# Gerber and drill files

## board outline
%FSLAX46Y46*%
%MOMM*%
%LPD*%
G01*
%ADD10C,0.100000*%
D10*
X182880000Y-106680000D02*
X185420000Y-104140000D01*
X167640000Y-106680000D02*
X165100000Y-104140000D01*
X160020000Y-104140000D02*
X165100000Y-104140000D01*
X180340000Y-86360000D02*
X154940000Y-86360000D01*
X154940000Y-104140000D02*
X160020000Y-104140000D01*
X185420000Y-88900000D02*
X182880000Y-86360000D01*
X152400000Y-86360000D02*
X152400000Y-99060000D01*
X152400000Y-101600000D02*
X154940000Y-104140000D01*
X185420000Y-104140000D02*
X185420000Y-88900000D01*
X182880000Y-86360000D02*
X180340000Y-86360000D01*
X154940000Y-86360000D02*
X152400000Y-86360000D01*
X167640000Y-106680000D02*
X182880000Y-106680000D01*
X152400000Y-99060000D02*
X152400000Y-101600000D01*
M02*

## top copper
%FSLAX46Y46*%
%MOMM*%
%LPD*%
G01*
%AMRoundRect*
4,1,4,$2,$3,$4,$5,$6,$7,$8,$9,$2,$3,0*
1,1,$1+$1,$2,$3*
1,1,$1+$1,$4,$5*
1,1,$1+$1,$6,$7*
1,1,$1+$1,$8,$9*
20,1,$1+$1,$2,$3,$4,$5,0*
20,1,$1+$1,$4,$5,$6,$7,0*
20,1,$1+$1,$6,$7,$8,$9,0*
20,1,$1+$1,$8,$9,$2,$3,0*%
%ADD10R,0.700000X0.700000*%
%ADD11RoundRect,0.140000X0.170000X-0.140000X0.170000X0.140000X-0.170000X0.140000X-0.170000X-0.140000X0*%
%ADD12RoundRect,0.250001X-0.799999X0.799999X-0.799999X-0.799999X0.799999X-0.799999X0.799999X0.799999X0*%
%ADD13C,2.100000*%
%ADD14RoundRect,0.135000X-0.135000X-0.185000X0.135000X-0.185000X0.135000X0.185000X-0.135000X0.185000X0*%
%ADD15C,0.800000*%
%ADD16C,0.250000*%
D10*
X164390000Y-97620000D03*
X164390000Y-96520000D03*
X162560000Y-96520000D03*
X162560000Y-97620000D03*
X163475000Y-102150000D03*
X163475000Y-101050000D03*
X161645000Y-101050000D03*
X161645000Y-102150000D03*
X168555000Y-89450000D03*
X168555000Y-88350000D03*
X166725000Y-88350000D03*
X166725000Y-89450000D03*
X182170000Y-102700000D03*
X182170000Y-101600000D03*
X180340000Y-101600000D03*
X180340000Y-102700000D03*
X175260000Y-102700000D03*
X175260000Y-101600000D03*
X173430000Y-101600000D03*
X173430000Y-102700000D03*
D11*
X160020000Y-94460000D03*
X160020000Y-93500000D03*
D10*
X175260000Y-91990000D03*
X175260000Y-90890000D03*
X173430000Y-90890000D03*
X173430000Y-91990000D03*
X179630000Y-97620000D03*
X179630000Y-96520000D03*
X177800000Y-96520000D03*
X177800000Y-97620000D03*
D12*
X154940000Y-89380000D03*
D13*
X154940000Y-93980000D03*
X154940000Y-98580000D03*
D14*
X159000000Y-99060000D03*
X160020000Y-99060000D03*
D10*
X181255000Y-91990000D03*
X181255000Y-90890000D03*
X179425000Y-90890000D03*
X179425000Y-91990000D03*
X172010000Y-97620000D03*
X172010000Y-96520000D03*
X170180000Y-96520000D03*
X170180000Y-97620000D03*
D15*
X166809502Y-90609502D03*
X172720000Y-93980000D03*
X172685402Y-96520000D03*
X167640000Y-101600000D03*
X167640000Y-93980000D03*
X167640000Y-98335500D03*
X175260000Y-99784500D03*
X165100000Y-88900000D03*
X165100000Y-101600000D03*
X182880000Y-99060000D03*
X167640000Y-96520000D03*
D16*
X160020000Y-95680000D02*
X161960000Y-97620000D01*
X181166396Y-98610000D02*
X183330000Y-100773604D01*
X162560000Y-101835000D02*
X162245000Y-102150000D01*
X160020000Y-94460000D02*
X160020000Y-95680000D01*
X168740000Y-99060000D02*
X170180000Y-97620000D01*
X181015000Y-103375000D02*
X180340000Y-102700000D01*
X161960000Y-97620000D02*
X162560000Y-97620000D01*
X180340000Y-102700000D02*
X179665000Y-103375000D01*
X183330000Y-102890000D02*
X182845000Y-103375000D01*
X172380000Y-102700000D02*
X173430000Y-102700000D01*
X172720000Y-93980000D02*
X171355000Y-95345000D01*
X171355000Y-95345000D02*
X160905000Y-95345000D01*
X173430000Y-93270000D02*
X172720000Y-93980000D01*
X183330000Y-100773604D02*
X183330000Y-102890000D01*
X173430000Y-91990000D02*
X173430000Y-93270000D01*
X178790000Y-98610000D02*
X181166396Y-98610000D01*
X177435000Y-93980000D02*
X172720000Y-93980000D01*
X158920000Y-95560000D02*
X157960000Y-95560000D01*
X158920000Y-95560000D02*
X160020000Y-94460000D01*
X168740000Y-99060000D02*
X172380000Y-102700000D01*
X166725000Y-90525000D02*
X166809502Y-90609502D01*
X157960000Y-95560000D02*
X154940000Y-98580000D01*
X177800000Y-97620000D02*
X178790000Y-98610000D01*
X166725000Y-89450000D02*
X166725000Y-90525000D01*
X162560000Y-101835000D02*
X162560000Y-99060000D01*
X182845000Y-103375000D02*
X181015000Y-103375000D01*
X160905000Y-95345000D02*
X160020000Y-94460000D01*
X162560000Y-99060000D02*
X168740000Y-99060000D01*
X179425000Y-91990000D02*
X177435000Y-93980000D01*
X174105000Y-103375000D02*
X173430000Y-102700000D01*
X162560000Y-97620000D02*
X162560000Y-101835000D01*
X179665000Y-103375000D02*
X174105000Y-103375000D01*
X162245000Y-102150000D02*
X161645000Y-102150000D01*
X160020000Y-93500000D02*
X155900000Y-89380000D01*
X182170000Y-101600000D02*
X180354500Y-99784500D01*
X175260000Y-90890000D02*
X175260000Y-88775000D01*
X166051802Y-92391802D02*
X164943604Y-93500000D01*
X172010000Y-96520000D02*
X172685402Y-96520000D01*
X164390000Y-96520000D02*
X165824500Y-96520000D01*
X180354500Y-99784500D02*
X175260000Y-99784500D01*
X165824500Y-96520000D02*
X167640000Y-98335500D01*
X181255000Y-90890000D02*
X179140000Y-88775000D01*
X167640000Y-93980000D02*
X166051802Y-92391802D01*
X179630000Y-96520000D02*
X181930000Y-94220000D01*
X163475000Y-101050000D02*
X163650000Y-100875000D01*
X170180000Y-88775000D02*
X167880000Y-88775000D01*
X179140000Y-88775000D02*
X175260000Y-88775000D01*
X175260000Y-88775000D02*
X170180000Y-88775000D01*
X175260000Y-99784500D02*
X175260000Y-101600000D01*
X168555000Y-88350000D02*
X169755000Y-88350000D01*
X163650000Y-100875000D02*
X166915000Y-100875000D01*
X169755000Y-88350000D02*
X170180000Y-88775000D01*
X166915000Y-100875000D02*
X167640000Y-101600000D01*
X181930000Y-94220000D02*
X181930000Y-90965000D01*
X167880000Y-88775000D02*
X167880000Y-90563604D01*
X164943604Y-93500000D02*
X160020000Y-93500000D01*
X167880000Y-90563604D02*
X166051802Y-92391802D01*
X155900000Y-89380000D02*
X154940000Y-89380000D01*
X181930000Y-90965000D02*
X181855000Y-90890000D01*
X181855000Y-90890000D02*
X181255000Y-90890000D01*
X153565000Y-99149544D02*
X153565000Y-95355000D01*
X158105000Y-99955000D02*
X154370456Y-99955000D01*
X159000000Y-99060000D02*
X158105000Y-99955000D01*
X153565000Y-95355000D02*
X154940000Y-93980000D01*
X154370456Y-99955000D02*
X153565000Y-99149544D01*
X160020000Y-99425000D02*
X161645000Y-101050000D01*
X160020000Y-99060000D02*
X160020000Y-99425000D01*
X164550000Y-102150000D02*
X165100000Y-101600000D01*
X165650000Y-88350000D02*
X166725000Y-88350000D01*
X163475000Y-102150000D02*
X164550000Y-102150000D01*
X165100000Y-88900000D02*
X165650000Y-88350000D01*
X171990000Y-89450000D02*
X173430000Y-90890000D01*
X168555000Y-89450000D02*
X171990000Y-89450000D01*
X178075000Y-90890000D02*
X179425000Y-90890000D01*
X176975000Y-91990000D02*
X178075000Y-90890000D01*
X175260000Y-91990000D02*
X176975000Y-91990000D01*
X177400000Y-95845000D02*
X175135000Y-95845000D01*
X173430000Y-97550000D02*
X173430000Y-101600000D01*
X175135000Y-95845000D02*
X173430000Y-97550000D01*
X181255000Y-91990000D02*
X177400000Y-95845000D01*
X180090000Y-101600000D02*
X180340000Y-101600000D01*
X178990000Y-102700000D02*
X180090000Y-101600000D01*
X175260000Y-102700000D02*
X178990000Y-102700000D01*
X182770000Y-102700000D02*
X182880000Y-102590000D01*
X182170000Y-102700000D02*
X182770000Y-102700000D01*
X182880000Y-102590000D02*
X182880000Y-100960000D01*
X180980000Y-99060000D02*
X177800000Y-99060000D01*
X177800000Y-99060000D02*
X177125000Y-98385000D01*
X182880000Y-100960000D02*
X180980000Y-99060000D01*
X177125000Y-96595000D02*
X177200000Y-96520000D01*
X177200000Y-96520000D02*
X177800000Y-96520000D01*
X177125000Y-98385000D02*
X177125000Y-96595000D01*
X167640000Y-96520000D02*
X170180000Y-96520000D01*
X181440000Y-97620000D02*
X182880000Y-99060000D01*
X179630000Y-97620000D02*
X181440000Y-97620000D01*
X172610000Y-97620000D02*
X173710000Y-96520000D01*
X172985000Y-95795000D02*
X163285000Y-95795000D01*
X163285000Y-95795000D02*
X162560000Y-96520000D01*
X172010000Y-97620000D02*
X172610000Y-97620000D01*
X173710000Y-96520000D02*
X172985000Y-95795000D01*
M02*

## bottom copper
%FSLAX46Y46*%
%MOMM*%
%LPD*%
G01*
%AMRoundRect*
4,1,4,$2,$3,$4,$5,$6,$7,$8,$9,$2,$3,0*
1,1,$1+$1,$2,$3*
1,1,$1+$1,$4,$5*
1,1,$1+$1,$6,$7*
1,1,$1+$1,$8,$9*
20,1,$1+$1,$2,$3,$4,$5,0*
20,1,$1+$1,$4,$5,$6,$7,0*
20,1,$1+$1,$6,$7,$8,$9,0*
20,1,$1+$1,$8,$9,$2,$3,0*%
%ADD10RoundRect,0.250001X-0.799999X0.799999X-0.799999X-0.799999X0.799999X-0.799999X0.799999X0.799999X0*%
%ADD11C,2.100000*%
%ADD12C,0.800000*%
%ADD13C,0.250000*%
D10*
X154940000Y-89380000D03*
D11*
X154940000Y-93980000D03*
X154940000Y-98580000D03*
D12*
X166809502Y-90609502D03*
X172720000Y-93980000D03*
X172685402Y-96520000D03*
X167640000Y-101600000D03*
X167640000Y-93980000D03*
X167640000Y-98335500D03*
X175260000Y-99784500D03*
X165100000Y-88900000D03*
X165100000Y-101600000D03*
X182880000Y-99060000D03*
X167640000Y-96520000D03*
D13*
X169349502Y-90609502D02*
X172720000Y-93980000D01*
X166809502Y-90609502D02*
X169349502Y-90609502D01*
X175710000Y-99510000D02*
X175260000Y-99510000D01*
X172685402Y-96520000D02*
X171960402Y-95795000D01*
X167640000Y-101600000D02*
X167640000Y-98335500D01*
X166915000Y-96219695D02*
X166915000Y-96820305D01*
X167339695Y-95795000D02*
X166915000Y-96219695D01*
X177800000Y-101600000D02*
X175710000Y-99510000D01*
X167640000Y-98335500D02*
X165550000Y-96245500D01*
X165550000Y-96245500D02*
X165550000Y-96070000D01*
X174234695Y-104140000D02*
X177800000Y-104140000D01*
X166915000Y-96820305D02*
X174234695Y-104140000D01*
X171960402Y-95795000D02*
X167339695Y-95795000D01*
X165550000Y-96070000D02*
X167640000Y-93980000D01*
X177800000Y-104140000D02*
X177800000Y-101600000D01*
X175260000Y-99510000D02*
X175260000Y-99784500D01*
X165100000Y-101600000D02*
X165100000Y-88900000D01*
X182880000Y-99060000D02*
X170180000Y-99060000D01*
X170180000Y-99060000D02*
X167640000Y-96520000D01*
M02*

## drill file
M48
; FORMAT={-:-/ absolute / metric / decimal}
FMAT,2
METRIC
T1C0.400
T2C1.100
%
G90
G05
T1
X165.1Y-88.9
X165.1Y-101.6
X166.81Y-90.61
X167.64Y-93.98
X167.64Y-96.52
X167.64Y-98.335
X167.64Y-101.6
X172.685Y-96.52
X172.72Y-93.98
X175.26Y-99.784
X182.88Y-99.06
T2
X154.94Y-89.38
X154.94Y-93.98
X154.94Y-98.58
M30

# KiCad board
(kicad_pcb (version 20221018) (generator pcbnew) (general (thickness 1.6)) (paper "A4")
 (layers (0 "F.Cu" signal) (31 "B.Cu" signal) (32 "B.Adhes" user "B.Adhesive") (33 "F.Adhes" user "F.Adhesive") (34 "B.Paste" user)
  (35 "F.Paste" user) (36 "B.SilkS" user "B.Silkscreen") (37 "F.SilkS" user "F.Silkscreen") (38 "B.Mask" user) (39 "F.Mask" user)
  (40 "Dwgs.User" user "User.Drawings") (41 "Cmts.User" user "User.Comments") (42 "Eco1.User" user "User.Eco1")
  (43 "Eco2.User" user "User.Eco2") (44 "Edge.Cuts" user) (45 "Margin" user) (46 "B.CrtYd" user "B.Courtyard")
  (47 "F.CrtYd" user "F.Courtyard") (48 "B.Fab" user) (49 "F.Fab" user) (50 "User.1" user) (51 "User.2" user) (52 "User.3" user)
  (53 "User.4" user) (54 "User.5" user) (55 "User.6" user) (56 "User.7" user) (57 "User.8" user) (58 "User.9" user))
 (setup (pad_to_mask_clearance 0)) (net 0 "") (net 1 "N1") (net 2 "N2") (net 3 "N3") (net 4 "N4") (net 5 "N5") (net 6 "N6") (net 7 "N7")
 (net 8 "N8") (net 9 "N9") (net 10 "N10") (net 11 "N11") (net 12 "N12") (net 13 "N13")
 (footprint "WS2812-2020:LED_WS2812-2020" (layer "F.Cu") (at 163.475 97.07)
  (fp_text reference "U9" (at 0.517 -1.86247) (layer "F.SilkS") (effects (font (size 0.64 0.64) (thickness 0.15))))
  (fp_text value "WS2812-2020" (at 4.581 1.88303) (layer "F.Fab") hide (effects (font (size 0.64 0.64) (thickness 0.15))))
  (pad "1" smd rect (at 0.915 0.55) (size 0.7 0.7) (layers "F.Cu" "F.Paste" "F.Mask") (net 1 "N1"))
  (pad "2" smd rect (at 0.915 -0.55) (size 0.7 0.7) (layers "F.Cu" "F.Paste" "F.Mask") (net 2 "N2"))
  (pad "3" smd rect (at -0.915 -0.55) (size 0.7 0.7) (layers "F.Cu" "F.Paste" "F.Mask") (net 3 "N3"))
  (pad "4" smd rect (at -0.915 0.55) (size 0.7 0.7) (layers "F.Cu" "F.Paste" "F.Mask") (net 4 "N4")))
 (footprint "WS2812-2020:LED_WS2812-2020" (layer "F.Cu") (at 162.56 101.6)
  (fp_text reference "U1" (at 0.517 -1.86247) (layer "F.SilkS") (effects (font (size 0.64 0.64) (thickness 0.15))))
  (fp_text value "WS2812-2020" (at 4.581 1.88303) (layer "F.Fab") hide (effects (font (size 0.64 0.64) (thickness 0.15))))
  (pad "1" smd rect (at 0.915 0.55) (size 0.7 0.7) (layers "F.Cu" "F.Paste" "F.Mask") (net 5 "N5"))
  (pad "2" smd rect (at 0.915 -0.55) (size 0.7 0.7) (layers "F.Cu" "F.Paste" "F.Mask") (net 2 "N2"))
  (pad "3" smd rect (at -0.915 -0.55) (size 0.7 0.7) (layers "F.Cu" "F.Paste" "F.Mask") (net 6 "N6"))
  (pad "4" smd rect (at -0.915 0.55) (size 0.7 0.7) (layers "F.Cu" "F.Paste" "F.Mask") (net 4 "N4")))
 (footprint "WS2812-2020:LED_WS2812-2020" (layer "F.Cu") (at 167.64 88.9)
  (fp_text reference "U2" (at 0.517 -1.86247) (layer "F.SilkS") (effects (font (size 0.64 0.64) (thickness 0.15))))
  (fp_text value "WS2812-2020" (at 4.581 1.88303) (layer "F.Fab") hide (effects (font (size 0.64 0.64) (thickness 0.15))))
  (pad "1" smd rect (at 0.915 0.55) (size 0.7 0.7) (layers "F.Cu" "F.Paste" "F.Mask") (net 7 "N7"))
  (pad "2" smd rect (at 0.915 -0.55) (size 0.7 0.7) (layers "F.Cu" "F.Paste" "F.Mask") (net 2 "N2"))
  (pad "3" smd rect (at -0.915 -0.55) (size 0.7 0.7) (layers "F.Cu" "F.Paste" "F.Mask") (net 5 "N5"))
  (pad "4" smd rect (at -0.915 0.55) (size 0.7 0.7) (layers "F.Cu" "F.Paste" "F.Mask") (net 4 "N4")))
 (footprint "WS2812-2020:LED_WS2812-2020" (layer "F.Cu") (at 181.255 102.15)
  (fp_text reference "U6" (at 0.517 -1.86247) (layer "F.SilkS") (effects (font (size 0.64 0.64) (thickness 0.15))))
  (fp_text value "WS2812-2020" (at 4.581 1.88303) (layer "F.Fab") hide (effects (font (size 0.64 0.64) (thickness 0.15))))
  (pad "1" smd rect (at 0.915 0.55) (size 0.7 0.7) (layers "F.Cu" "F.Paste" "F.Mask") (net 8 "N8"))
  (pad "2" smd rect (at 0.915 -0.55) (size 0.7 0.7) (layers "F.Cu" "F.Paste" "F.Mask") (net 2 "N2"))
  (pad "3" smd rect (at -0.915 -0.55) (size 0.7 0.7) (layers "F.Cu" "F.Paste" "F.Mask") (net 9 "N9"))
  (pad "4" smd rect (at -0.915 0.55) (size 0.7 0.7) (layers "F.Cu" "F.Paste" "F.Mask") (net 4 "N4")))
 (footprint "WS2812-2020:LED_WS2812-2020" (layer "F.Cu") (at 174.345 102.15)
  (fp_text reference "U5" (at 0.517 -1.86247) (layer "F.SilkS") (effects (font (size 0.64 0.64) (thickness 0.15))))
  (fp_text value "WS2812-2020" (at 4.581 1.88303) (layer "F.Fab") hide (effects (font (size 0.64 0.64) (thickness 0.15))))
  (pad "1" smd rect (at 0.915 0.55) (size 0.7 0.7) (layers "F.Cu" "F.Paste" "F.Mask") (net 9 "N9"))
  (pad "2" smd rect (at 0.915 -0.55) (size 0.7 0.7) (layers "F.Cu" "F.Paste" "F.Mask") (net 2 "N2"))
  (pad "3" smd rect (at -0.915 -0.55) (size 0.7 0.7) (layers "F.Cu" "F.Paste" "F.Mask") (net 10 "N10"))
  (pad "4" smd rect (at -0.915 0.55) (size 0.7 0.7) (layers "F.Cu" "F.Paste" "F.Mask") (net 4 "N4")))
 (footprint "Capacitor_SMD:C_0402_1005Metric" (layer "F.Cu") (at 160.02 93.98 90)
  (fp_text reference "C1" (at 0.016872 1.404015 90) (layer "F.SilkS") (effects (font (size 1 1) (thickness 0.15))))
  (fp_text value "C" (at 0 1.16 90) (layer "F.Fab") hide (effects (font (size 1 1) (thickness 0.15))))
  (pad "1" smd roundrect (at -0.48 0 90) (size 0.56 0.62) (layers "F.Cu" "F.Paste" "F.Mask") (roundrect_rratio 0.25) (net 4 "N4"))
  (pad "2" smd roundrect (at 0.48 0 90) (size 0.56 0.62) (layers "F.Cu" "F.Paste" "F.Mask") (roundrect_rratio 0.25) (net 2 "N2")))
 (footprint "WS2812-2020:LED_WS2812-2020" (layer "F.Cu") (at 174.345 91.44)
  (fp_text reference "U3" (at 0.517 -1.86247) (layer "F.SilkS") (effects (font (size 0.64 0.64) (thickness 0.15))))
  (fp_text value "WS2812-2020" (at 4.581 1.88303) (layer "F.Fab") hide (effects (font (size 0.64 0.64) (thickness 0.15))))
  (pad "1" smd rect (at 0.915 0.55) (size 0.7 0.7) (layers "F.Cu" "F.Paste" "F.Mask") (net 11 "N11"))
  (pad "2" smd rect (at 0.915 -0.55) (size 0.7 0.7) (layers "F.Cu" "F.Paste" "F.Mask") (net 2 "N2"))
  (pad "3" smd rect (at -0.915 -0.55) (size 0.7 0.7) (layers "F.Cu" "F.Paste" "F.Mask") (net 7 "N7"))
  (pad "4" smd rect (at -0.915 0.55) (size 0.7 0.7) (layers "F.Cu" "F.Paste" "F.Mask") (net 4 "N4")))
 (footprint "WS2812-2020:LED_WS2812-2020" (layer "F.Cu") (at 178.715 97.07)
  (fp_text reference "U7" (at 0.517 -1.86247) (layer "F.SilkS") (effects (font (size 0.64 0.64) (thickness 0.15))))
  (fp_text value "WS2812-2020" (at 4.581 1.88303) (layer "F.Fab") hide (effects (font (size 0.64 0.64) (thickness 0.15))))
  (pad "1" smd rect (at 0.915 0.55) (size 0.7 0.7) (layers "F.Cu" "F.Paste" "F.Mask") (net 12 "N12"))
  (pad "2" smd rect (at 0.915 -0.55) (size 0.7 0.7) (layers "F.Cu" "F.Paste" "F.Mask") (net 2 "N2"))
  (pad "3" smd rect (at -0.915 -0.55) (size 0.7 0.7) (layers "F.Cu" "F.Paste" "F.Mask") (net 8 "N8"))
  (pad "4" smd rect (at -0.915 0.55) (size 0.7 0.7) (layers "F.Cu" "F.Paste" "F.Mask") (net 4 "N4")))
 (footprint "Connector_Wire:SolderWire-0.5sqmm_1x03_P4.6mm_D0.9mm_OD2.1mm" (layer "F.Cu") (at 154.94 89.38 -90)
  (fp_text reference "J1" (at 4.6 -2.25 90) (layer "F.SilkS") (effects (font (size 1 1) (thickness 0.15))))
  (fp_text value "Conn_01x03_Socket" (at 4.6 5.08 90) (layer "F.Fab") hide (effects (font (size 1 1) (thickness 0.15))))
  (pad "1" thru_hole roundrect (at 0 0 270) (size 2.1 2.1) (drill 1.1) (layers "*.Cu" "*.Mask") (roundrect_rratio 0.119048) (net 2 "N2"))
  (pad "2" thru_hole circle (at 4.6 0 270) (size 2.1 2.1) (drill 1.1) (layers "*.Cu" "*.Mask") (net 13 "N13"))
  (pad "3" thru_hole circle (at 9.2 0 270) (size 2.1 2.1) (drill 1.1) (layers "*.Cu" "*.Mask") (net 4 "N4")))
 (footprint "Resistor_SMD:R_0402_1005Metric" (layer "F.Cu") (at 159.51 99.06)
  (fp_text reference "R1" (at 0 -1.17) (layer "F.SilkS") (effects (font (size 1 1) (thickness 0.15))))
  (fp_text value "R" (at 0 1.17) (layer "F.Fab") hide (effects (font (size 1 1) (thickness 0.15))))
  (pad "1" smd roundrect (at -0.51 0) (size 0.54 0.64) (layers "F.Cu" "F.Paste" "F.Mask") (roundrect_rratio 0.25) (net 13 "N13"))
  (pad "2" smd roundrect (at 0.51 0) (size 0.54 0.64) (layers "F.Cu" "F.Paste" "F.Mask") (roundrect_rratio 0.25) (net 6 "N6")))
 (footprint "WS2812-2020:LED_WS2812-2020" (layer "F.Cu") (at 180.34 91.44)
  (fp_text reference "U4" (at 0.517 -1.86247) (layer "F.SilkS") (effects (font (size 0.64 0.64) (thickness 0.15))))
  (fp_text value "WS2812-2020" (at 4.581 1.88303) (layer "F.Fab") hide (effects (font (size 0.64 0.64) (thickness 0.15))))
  (pad "1" smd rect (at 0.915 0.55) (size 0.7 0.7) (layers "F.Cu" "F.Paste" "F.Mask") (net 10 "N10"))
  (pad "2" smd rect (at 0.915 -0.55) (size 0.7 0.7) (layers "F.Cu" "F.Paste" "F.Mask") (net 2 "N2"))
  (pad "3" smd rect (at -0.915 -0.55) (size 0.7 0.7) (layers "F.Cu" "F.Paste" "F.Mask") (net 11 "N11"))
  (pad "4" smd rect (at -0.915 0.55) (size 0.7 0.7) (layers "F.Cu" "F.Paste" "F.Mask") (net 4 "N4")))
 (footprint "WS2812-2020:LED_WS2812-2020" (layer "F.Cu") (at 171.095 97.07)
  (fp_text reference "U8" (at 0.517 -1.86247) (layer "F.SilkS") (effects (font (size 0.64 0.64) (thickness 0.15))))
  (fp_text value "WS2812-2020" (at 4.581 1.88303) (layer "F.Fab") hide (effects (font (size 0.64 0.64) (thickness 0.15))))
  (pad "1" smd rect (at 0.915 0.55) (size 0.7 0.7) (layers "F.Cu" "F.Paste" "F.Mask") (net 3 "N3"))
  (pad "2" smd rect (at 0.915 -0.55) (size 0.7 0.7) (layers "F.Cu" "F.Paste" "F.Mask") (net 2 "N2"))
  (pad "3" smd rect (at -0.915 -0.55) (size 0.7 0.7) (layers "F.Cu" "F.Paste" "F.Mask") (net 12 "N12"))
  (pad "4" smd rect (at -0.915 0.55) (size 0.7 0.7) (layers "F.Cu" "F.Paste" "F.Mask") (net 4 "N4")))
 (gr_line (start 182.88 106.68) (end 185.42 104.14) (stroke (width 0.1) (type default)) (layer "Edge.Cuts"))
 (gr_line (start 167.64 106.68) (end 165.1 104.14) (stroke (width 0.1) (type default)) (layer "Edge.Cuts"))
 (gr_line (start 160.02 104.14) (end 165.1 104.14) (stroke (width 0.1) (type default)) (layer "Edge.Cuts"))
 (gr_line (start 180.34 86.36) (end 154.94 86.36) (stroke (width 0.1) (type default)) (layer "Edge.Cuts"))
 (gr_line (start 154.94 104.14) (end 160.02 104.14) (stroke (width 0.1) (type default)) (layer "Edge.Cuts"))
 (gr_line (start 185.42 88.9) (end 182.88 86.36) (stroke (width 0.1) (type default)) (layer "Edge.Cuts"))
 (gr_line (start 152.4 86.36) (end 152.4 99.06) (stroke (width 0.1) (type default)) (layer "Edge.Cuts"))
 (gr_line (start 152.4 101.6) (end 154.94 104.14) (stroke (width 0.1) (type default)) (layer "Edge.Cuts"))
 (gr_line (start 185.42 104.14) (end 185.42 88.9) (stroke (width 0.1) (type default)) (layer "Edge.Cuts"))
 (gr_line (start 182.88 86.36) (end 180.34 86.36) (stroke (width 0.1) (type default)) (layer "Edge.Cuts"))
 (gr_line (start 154.94 86.36) (end 152.4 86.36) (stroke (width 0.1) (type default)) (layer "Edge.Cuts"))
 (gr_line (start 167.64 106.68) (end 182.88 106.68) (stroke (width 0.1) (type default)) (layer "Edge.Cuts"))
 (gr_line (start 152.4 99.06) (end 152.4 101.6) (stroke (width 0.1) (type default)) (layer "Edge.Cuts"))
 (segment (start 160.02 95.68) (end 161.96 97.62) (width 0.25) (layer "F.Cu") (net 4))
 (segment (start 181.166396 98.61) (end 183.33 100.773604) (width 0.25) (layer "F.Cu") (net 4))
 (segment (start 162.56 101.835) (end 162.245 102.15) (width 0.25) (layer "F.Cu") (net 4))
 (segment (start 160.02 94.46) (end 160.02 95.68) (width 0.25) (layer "F.Cu") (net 4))
 (segment (start 168.74 99.06) (end 170.18 97.62) (width 0.25) (layer "F.Cu") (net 4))
 (segment (start 181.015 103.375) (end 180.34 102.7) (width 0.25) (layer "F.Cu") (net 4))
 (segment (start 161.96 97.62) (end 162.56 97.62) (width 0.25) (layer "F.Cu") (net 4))
 (segment (start 180.34 102.7) (end 179.665 103.375) (width 0.25) (layer "F.Cu") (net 4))
 (segment (start 183.33 102.89) (end 182.845 103.375) (width 0.25) (layer "F.Cu") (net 4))
 (segment (start 172.38 102.7) (end 173.43 102.7) (width 0.25) (layer "F.Cu") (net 4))
 (segment (start 172.72 93.98) (end 171.355 95.345) (width 0.25) (layer "F.Cu") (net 4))
 (segment (start 171.355 95.345) (end 160.905 95.345) (width 0.25) (layer "F.Cu") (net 4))
 (segment (start 173.43 93.27) (end 172.72 93.98) (width 0.25) (layer "F.Cu") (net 4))
 (segment (start 183.33 100.773604) (end 183.33 102.89) (width 0.25) (layer "F.Cu") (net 4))
 (segment (start 173.43 91.99) (end 173.43 93.27) (width 0.25) (layer "F.Cu") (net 4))
 (segment (start 178.79 98.61) (end 181.166396 98.61) (width 0.25) (layer "F.Cu") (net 4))
 (segment (start 177.435 93.98) (end 172.72 93.98) (width 0.25) (layer "F.Cu") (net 4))
 (segment (start 158.92 95.56) (end 157.96 95.56) (width 0.25) (layer "F.Cu") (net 4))
 (segment (start 158.92 95.56) (end 160.02 94.46) (width 0.25) (layer "F.Cu") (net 4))
 (segment (start 168.74 99.06) (end 172.38 102.7) (width 0.25) (layer "F.Cu") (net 4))
 (segment (start 166.725 90.525) (end 166.809502 90.609502) (width 0.25) (layer "F.Cu") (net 4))
 (segment (start 157.96 95.56) (end 154.94 98.58) (width 0.25) (layer "F.Cu") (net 4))
 (segment (start 177.8 97.62) (end 178.79 98.61) (width 0.25) (layer "F.Cu") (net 4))
 (segment (start 166.725 89.45) (end 166.725 90.525) (width 0.25) (layer "F.Cu") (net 4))
 (segment (start 162.56 101.835) (end 162.56 99.06) (width 0.25) (layer "F.Cu") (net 4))
 (segment (start 182.845 103.375) (end 181.015 103.375) (width 0.25) (layer "F.Cu") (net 4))
 (segment (start 160.905 95.345) (end 160.02 94.46) (width 0.25) (layer "F.Cu") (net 4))
 (segment (start 162.56 99.06) (end 168.74 99.06) (width 0.25) (layer "F.Cu") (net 4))
 (segment (start 179.425 91.99) (end 177.435 93.98) (width 0.25) (layer "F.Cu") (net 4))
 (segment (start 174.105 103.375) (end 173.43 102.7) (width 0.25) (layer "F.Cu") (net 4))
 (segment (start 162.56 97.62) (end 162.56 101.835) (width 0.25) (layer "F.Cu") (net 4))
 (segment (start 179.665 103.375) (end 174.105 103.375) (width 0.25) (layer "F.Cu") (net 4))
 (segment (start 162.245 102.15) (end 161.645 102.15) (width 0.25) (layer "F.Cu") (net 4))
 (via (at 166.809502 90.609502) (size 0.8) (drill 0.4) (layers "F.Cu" "B.Cu") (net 4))
 (via (at 172.72 93.98) (size 0.8) (drill 0.4) (layers "F.Cu" "B.Cu") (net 4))
 (segment (start 169.349502 90.609502) (end 172.72 93.98) (width 0.25) (layer "B.Cu") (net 4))
 (segment (start 166.809502 90.609502) (end 169.349502 90.609502) (width 0.25) (layer "B.Cu") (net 4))
 (segment (start 160.02 93.5) (end 155.9 89.38) (width 0.25) (layer "F.Cu") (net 2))
 (segment (start 182.17 101.6) (end 180.3545 99.7845) (width 0.25) (layer "F.Cu") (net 2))
 (segment (start 175.26 90.89) (end 175.26 88.775) (width 0.25) (layer "F.Cu") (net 2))
 (segment (start 166.051802 92.391802) (end 164.943604 93.5) (width 0.25) (layer "F.Cu") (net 2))
 (segment (start 172.01 96.52) (end 172.685402 96.52) (width 0.25) (layer "F.Cu") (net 2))
 (segment (start 164.39 96.52) (end 165.8245 96.52) (width 0.25) (layer "F.Cu") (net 2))
 (segment (start 180.3545 99.7845) (end 175.26 99.7845) (width 0.25) (layer "F.Cu") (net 2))
 (segment (start 165.8245 96.52) (end 167.64 98.3355) (width 0.25) (layer "F.Cu") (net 2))
 (segment (start 181.255 90.89) (end 179.14 88.775) (width 0.25) (layer "F.Cu") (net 2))
 (segment (start 167.64 93.98) (end 166.051802 92.391802) (width 0.25) (layer "F.Cu") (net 2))
 (segment (start 179.63 96.52) (end 181.93 94.22) (width 0.25) (layer "F.Cu") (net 2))
 (segment (start 163.475 101.05) (end 163.65 100.875) (width 0.25) (layer "F.Cu") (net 2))
 (segment (start 170.18 88.775) (end 167.88 88.775) (width 0.25) (layer "F.Cu") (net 2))
 (segment (start 179.14 88.775) (end 175.26 88.775) (width 0.25) (layer "F.Cu") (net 2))
 (segment (start 175.26 88.775) (end 170.18 88.775) (width 0.25) (layer "F.Cu") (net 2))
 (segment (start 175.26 99.7845) (end 175.26 101.6) (width 0.25) (layer "F.Cu") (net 2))
 (segment (start 168.555 88.35) (end 169.755 88.35) (width 0.25) (layer "F.Cu") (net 2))
 (segment (start 163.65 100.875) (end 166.915 100.875) (width 0.25) (layer "F.Cu") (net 2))
 (segment (start 169.755 88.35) (end 170.18 88.775) (width 0.25) (layer "F.Cu") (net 2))
 (segment (start 166.915 100.875) (end 167.64 101.6) (width 0.25) (layer "F.Cu") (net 2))
 (segment (start 181.93 94.22) (end 181.93 90.965) (width 0.25) (layer "F.Cu") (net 2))
 (segment (start 167.88 88.775) (end 167.88 90.563604) (width 0.25) (layer "F.Cu") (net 2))
 (segment (start 164.943604 93.5) (end 160.02 93.5) (width 0.25) (layer "F.Cu") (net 2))
 (segment (start 167.88 90.563604) (end 166.051802 92.391802) (width 0.25) (layer "F.Cu") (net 2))
 (segment (start 155.9 89.38) (end 154.94 89.38) (width 0.25) (layer "F.Cu") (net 2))
 (segment (start 181.93 90.965) (end 181.855 90.89) (width 0.25) (layer "F.Cu") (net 2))
 (segment (start 181.855 90.89) (end 181.255 90.89) (width 0.25) (layer "F.Cu") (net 2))
 (via (at 172.685402 96.52) (size 0.8) (drill 0.4) (layers "F.Cu" "B.Cu") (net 2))
 (via (at 167.64 101.6) (size 0.8) (drill 0.4) (layers "F.Cu" "B.Cu") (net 2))
 (via (at 167.64 93.98) (size 0.8) (drill 0.4) (layers "F.Cu" "B.Cu") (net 2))
 (via (at 167.64 98.3355) (size 0.8) (drill 0.4) (layers "F.Cu" "B.Cu") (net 2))
 (via (at 175.26 99.7845) (size 0.8) (drill 0.4) (layers "F.Cu" "B.Cu") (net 2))
 (segment (start 175.71 99.51) (end 175.26 99.51) (width 0.25) (layer "B.Cu") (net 2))
 (segment (start 172.685402 96.52) (end 171.960402 95.795) (width 0.25) (layer "B.Cu") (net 2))
 (segment (start 167.64 101.6) (end 167.64 98.3355) (width 0.25) (layer "B.Cu") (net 2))
 (segment (start 166.915 96.219695) (end 166.915 96.820305) (width 0.25) (layer "B.Cu") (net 2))
 (segment (start 167.339695 95.795) (end 166.915 96.219695) (width 0.25) (layer "B.Cu") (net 2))
 (segment (start 177.8 101.6) (end 175.71 99.51) (width 0.25) (layer "B.Cu") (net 2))
 (segment (start 167.64 98.3355) (end 165.55 96.2455) (width 0.25) (layer "B.Cu") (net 2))
 (segment (start 165.55 96.2455) (end 165.55 96.07) (width 0.25) (layer "B.Cu") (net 2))
 (segment (start 174.234695 104.14) (end 177.8 104.14) (width 0.25) (layer "B.Cu") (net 2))
 (segment (start 166.915 96.820305) (end 174.234695 104.14) (width 0.25) (layer "B.Cu") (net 2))
 (segment (start 171.960402 95.795) (end 167.339695 95.795) (width 0.25) (layer "B.Cu") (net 2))
 (segment (start 165.55 96.07) (end 167.64 93.98) (width 0.25) (layer "B.Cu") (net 2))
 (segment (start 177.8 104.14) (end 177.8 101.6) (width 0.25) (layer "B.Cu") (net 2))
 (segment (start 175.26 99.51) (end 175.26 99.7845) (width 0.25) (layer "B.Cu") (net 2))
 (segment (start 153.565 99.149544) (end 153.565 95.355) (width 0.25) (layer "F.Cu") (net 13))
 (segment (start 158.105 99.955) (end 154.370456 99.955) (width 0.25) (layer "F.Cu") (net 13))
 (segment (start 159 99.06) (end 158.105 99.955) (width 0.25) (layer "F.Cu") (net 13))
 (segment (start 153.565 95.355) (end 154.94 93.98) (width 0.25) (layer "F.Cu") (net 13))
 (segment (start 154.370456 99.955) (end 153.565 99.149544) (width 0.25) (layer "F.Cu") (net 13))
 (segment (start 160.02 99.425) (end 161.645 101.05) (width 0.25) (layer "F.Cu") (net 6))
 (segment (start 160.02 99.06) (end 160.02 99.425) (width 0.25) (layer "F.Cu") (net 6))
 (segment (start 164.55 102.15) (end 165.1 101.6) (width 0.25) (layer "F.Cu") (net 5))
 (segment (start 165.65 88.35) (end 166.725 88.35) (width 0.25) (layer "F.Cu") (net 5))
 (segment (start 163.475 102.15) (end 164.55 102.15) (width 0.25) (layer "F.Cu") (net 5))
 (segment (start 165.1 88.9) (end 165.65 88.35) (width 0.25) (layer "F.Cu") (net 5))
 (via (at 165.1 88.9) (size 0.8) (drill 0.4) (layers "F.Cu" "B.Cu") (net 5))
 (via (at 165.1 101.6) (size 0.8) (drill 0.4) (layers "F.Cu" "B.Cu") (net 5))
 (segment (start 165.1 101.6) (end 165.1 88.9) (width 0.25) (layer "B.Cu") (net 5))
 (segment (start 171.99 89.45) (end 173.43 90.89) (width 0.25) (layer "F.Cu") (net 7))
 (segment (start 168.555 89.45) (end 171.99 89.45) (width 0.25) (layer "F.Cu") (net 7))
 (segment (start 178.075 90.89) (end 179.425 90.89) (width 0.25) (layer "F.Cu") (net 11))
 (segment (start 176.975 91.99) (end 178.075 90.89) (width 0.25) (layer "F.Cu") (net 11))
 (segment (start 175.26 91.99) (end 176.975 91.99) (width 0.25) (layer "F.Cu") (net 11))
 (segment (start 177.4 95.845) (end 175.135 95.845) (width 0.25) (layer "F.Cu") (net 10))
 (segment (start 173.43 97.55) (end 173.43 101.6) (width 0.25) (layer "F.Cu") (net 10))
 (segment (start 175.135 95.845) (end 173.43 97.55) (width 0.25) (layer "F.Cu") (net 10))
 (segment (start 181.255 91.99) (end 177.4 95.845) (width 0.25) (layer "F.Cu") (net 10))
 (segment (start 180.09 101.6) (end 180.34 101.6) (width 0.25) (layer "F.Cu") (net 9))
 (segment (start 178.99 102.7) (end 180.09 101.6) (width 0.25) (layer "F.Cu") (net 9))
 (segment (start 175.26 102.7) (end 178.99 102.7) (width 0.25) (layer "F.Cu") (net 9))
 (segment (start 182.77 102.7) (end 182.88 102.59) (width 0.25) (layer "F.Cu") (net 8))
 (segment (start 182.17 102.7) (end 182.77 102.7) (width 0.25) (layer "F.Cu") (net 8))
 (segment (start 182.88 102.59) (end 182.88 100.96) (width 0.25) (layer "F.Cu") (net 8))
 (segment (start 180.98 99.06) (end 177.8 99.06) (width 0.25) (layer "F.Cu") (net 8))
 (segment (start 177.8 99.06) (end 177.125 98.385) (width 0.25) (layer "F.Cu") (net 8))
 (segment (start 182.88 100.96) (end 180.98 99.06) (width 0.25) (layer "F.Cu") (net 8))
 (segment (start 177.125 96.595) (end 177.2 96.52) (width 0.25) (layer "F.Cu") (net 8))
 (segment (start 177.2 96.52) (end 177.8 96.52) (width 0.25) (layer "F.Cu") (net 8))
 (segment (start 177.125 98.385) (end 177.125 96.595) (width 0.25) (layer "F.Cu") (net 8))
 (segment (start 167.64 96.52) (end 170.18 96.52) (width 0.25) (layer "F.Cu") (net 12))
 (segment (start 181.44 97.62) (end 182.88 99.06) (width 0.25) (layer "F.Cu") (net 12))
 (segment (start 179.63 97.62) (end 181.44 97.62) (width 0.25) (layer "F.Cu") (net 12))
 (via (at 182.88 99.06) (size 0.8) (drill 0.4) (layers "F.Cu" "B.Cu") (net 12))
 (via (at 167.64 96.52) (size 0.8) (drill 0.4) (layers "F.Cu" "B.Cu") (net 12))
 (segment (start 182.88 99.06) (end 170.18 99.06) (width 0.25) (layer "B.Cu") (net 12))
 (segment (start 170.18 99.06) (end 167.64 96.52) (width 0.25) (layer "B.Cu") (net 12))
 (segment (start 172.61 97.62) (end 173.71 96.52) (width 0.25) (layer "F.Cu") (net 3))
 (segment (start 172.985 95.795) (end 163.285 95.795) (width 0.25) (layer "F.Cu") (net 3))
 (segment (start 163.285 95.795) (end 162.56 96.52) (width 0.25) (layer "F.Cu") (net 3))
 (segment (start 172.01 97.62) (end 172.61 97.62) (width 0.25) (layer "F.Cu") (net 3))
 (segment (start 173.71 96.52) (end 172.985 95.795) (width 0.25) (layer "F.Cu") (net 3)))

